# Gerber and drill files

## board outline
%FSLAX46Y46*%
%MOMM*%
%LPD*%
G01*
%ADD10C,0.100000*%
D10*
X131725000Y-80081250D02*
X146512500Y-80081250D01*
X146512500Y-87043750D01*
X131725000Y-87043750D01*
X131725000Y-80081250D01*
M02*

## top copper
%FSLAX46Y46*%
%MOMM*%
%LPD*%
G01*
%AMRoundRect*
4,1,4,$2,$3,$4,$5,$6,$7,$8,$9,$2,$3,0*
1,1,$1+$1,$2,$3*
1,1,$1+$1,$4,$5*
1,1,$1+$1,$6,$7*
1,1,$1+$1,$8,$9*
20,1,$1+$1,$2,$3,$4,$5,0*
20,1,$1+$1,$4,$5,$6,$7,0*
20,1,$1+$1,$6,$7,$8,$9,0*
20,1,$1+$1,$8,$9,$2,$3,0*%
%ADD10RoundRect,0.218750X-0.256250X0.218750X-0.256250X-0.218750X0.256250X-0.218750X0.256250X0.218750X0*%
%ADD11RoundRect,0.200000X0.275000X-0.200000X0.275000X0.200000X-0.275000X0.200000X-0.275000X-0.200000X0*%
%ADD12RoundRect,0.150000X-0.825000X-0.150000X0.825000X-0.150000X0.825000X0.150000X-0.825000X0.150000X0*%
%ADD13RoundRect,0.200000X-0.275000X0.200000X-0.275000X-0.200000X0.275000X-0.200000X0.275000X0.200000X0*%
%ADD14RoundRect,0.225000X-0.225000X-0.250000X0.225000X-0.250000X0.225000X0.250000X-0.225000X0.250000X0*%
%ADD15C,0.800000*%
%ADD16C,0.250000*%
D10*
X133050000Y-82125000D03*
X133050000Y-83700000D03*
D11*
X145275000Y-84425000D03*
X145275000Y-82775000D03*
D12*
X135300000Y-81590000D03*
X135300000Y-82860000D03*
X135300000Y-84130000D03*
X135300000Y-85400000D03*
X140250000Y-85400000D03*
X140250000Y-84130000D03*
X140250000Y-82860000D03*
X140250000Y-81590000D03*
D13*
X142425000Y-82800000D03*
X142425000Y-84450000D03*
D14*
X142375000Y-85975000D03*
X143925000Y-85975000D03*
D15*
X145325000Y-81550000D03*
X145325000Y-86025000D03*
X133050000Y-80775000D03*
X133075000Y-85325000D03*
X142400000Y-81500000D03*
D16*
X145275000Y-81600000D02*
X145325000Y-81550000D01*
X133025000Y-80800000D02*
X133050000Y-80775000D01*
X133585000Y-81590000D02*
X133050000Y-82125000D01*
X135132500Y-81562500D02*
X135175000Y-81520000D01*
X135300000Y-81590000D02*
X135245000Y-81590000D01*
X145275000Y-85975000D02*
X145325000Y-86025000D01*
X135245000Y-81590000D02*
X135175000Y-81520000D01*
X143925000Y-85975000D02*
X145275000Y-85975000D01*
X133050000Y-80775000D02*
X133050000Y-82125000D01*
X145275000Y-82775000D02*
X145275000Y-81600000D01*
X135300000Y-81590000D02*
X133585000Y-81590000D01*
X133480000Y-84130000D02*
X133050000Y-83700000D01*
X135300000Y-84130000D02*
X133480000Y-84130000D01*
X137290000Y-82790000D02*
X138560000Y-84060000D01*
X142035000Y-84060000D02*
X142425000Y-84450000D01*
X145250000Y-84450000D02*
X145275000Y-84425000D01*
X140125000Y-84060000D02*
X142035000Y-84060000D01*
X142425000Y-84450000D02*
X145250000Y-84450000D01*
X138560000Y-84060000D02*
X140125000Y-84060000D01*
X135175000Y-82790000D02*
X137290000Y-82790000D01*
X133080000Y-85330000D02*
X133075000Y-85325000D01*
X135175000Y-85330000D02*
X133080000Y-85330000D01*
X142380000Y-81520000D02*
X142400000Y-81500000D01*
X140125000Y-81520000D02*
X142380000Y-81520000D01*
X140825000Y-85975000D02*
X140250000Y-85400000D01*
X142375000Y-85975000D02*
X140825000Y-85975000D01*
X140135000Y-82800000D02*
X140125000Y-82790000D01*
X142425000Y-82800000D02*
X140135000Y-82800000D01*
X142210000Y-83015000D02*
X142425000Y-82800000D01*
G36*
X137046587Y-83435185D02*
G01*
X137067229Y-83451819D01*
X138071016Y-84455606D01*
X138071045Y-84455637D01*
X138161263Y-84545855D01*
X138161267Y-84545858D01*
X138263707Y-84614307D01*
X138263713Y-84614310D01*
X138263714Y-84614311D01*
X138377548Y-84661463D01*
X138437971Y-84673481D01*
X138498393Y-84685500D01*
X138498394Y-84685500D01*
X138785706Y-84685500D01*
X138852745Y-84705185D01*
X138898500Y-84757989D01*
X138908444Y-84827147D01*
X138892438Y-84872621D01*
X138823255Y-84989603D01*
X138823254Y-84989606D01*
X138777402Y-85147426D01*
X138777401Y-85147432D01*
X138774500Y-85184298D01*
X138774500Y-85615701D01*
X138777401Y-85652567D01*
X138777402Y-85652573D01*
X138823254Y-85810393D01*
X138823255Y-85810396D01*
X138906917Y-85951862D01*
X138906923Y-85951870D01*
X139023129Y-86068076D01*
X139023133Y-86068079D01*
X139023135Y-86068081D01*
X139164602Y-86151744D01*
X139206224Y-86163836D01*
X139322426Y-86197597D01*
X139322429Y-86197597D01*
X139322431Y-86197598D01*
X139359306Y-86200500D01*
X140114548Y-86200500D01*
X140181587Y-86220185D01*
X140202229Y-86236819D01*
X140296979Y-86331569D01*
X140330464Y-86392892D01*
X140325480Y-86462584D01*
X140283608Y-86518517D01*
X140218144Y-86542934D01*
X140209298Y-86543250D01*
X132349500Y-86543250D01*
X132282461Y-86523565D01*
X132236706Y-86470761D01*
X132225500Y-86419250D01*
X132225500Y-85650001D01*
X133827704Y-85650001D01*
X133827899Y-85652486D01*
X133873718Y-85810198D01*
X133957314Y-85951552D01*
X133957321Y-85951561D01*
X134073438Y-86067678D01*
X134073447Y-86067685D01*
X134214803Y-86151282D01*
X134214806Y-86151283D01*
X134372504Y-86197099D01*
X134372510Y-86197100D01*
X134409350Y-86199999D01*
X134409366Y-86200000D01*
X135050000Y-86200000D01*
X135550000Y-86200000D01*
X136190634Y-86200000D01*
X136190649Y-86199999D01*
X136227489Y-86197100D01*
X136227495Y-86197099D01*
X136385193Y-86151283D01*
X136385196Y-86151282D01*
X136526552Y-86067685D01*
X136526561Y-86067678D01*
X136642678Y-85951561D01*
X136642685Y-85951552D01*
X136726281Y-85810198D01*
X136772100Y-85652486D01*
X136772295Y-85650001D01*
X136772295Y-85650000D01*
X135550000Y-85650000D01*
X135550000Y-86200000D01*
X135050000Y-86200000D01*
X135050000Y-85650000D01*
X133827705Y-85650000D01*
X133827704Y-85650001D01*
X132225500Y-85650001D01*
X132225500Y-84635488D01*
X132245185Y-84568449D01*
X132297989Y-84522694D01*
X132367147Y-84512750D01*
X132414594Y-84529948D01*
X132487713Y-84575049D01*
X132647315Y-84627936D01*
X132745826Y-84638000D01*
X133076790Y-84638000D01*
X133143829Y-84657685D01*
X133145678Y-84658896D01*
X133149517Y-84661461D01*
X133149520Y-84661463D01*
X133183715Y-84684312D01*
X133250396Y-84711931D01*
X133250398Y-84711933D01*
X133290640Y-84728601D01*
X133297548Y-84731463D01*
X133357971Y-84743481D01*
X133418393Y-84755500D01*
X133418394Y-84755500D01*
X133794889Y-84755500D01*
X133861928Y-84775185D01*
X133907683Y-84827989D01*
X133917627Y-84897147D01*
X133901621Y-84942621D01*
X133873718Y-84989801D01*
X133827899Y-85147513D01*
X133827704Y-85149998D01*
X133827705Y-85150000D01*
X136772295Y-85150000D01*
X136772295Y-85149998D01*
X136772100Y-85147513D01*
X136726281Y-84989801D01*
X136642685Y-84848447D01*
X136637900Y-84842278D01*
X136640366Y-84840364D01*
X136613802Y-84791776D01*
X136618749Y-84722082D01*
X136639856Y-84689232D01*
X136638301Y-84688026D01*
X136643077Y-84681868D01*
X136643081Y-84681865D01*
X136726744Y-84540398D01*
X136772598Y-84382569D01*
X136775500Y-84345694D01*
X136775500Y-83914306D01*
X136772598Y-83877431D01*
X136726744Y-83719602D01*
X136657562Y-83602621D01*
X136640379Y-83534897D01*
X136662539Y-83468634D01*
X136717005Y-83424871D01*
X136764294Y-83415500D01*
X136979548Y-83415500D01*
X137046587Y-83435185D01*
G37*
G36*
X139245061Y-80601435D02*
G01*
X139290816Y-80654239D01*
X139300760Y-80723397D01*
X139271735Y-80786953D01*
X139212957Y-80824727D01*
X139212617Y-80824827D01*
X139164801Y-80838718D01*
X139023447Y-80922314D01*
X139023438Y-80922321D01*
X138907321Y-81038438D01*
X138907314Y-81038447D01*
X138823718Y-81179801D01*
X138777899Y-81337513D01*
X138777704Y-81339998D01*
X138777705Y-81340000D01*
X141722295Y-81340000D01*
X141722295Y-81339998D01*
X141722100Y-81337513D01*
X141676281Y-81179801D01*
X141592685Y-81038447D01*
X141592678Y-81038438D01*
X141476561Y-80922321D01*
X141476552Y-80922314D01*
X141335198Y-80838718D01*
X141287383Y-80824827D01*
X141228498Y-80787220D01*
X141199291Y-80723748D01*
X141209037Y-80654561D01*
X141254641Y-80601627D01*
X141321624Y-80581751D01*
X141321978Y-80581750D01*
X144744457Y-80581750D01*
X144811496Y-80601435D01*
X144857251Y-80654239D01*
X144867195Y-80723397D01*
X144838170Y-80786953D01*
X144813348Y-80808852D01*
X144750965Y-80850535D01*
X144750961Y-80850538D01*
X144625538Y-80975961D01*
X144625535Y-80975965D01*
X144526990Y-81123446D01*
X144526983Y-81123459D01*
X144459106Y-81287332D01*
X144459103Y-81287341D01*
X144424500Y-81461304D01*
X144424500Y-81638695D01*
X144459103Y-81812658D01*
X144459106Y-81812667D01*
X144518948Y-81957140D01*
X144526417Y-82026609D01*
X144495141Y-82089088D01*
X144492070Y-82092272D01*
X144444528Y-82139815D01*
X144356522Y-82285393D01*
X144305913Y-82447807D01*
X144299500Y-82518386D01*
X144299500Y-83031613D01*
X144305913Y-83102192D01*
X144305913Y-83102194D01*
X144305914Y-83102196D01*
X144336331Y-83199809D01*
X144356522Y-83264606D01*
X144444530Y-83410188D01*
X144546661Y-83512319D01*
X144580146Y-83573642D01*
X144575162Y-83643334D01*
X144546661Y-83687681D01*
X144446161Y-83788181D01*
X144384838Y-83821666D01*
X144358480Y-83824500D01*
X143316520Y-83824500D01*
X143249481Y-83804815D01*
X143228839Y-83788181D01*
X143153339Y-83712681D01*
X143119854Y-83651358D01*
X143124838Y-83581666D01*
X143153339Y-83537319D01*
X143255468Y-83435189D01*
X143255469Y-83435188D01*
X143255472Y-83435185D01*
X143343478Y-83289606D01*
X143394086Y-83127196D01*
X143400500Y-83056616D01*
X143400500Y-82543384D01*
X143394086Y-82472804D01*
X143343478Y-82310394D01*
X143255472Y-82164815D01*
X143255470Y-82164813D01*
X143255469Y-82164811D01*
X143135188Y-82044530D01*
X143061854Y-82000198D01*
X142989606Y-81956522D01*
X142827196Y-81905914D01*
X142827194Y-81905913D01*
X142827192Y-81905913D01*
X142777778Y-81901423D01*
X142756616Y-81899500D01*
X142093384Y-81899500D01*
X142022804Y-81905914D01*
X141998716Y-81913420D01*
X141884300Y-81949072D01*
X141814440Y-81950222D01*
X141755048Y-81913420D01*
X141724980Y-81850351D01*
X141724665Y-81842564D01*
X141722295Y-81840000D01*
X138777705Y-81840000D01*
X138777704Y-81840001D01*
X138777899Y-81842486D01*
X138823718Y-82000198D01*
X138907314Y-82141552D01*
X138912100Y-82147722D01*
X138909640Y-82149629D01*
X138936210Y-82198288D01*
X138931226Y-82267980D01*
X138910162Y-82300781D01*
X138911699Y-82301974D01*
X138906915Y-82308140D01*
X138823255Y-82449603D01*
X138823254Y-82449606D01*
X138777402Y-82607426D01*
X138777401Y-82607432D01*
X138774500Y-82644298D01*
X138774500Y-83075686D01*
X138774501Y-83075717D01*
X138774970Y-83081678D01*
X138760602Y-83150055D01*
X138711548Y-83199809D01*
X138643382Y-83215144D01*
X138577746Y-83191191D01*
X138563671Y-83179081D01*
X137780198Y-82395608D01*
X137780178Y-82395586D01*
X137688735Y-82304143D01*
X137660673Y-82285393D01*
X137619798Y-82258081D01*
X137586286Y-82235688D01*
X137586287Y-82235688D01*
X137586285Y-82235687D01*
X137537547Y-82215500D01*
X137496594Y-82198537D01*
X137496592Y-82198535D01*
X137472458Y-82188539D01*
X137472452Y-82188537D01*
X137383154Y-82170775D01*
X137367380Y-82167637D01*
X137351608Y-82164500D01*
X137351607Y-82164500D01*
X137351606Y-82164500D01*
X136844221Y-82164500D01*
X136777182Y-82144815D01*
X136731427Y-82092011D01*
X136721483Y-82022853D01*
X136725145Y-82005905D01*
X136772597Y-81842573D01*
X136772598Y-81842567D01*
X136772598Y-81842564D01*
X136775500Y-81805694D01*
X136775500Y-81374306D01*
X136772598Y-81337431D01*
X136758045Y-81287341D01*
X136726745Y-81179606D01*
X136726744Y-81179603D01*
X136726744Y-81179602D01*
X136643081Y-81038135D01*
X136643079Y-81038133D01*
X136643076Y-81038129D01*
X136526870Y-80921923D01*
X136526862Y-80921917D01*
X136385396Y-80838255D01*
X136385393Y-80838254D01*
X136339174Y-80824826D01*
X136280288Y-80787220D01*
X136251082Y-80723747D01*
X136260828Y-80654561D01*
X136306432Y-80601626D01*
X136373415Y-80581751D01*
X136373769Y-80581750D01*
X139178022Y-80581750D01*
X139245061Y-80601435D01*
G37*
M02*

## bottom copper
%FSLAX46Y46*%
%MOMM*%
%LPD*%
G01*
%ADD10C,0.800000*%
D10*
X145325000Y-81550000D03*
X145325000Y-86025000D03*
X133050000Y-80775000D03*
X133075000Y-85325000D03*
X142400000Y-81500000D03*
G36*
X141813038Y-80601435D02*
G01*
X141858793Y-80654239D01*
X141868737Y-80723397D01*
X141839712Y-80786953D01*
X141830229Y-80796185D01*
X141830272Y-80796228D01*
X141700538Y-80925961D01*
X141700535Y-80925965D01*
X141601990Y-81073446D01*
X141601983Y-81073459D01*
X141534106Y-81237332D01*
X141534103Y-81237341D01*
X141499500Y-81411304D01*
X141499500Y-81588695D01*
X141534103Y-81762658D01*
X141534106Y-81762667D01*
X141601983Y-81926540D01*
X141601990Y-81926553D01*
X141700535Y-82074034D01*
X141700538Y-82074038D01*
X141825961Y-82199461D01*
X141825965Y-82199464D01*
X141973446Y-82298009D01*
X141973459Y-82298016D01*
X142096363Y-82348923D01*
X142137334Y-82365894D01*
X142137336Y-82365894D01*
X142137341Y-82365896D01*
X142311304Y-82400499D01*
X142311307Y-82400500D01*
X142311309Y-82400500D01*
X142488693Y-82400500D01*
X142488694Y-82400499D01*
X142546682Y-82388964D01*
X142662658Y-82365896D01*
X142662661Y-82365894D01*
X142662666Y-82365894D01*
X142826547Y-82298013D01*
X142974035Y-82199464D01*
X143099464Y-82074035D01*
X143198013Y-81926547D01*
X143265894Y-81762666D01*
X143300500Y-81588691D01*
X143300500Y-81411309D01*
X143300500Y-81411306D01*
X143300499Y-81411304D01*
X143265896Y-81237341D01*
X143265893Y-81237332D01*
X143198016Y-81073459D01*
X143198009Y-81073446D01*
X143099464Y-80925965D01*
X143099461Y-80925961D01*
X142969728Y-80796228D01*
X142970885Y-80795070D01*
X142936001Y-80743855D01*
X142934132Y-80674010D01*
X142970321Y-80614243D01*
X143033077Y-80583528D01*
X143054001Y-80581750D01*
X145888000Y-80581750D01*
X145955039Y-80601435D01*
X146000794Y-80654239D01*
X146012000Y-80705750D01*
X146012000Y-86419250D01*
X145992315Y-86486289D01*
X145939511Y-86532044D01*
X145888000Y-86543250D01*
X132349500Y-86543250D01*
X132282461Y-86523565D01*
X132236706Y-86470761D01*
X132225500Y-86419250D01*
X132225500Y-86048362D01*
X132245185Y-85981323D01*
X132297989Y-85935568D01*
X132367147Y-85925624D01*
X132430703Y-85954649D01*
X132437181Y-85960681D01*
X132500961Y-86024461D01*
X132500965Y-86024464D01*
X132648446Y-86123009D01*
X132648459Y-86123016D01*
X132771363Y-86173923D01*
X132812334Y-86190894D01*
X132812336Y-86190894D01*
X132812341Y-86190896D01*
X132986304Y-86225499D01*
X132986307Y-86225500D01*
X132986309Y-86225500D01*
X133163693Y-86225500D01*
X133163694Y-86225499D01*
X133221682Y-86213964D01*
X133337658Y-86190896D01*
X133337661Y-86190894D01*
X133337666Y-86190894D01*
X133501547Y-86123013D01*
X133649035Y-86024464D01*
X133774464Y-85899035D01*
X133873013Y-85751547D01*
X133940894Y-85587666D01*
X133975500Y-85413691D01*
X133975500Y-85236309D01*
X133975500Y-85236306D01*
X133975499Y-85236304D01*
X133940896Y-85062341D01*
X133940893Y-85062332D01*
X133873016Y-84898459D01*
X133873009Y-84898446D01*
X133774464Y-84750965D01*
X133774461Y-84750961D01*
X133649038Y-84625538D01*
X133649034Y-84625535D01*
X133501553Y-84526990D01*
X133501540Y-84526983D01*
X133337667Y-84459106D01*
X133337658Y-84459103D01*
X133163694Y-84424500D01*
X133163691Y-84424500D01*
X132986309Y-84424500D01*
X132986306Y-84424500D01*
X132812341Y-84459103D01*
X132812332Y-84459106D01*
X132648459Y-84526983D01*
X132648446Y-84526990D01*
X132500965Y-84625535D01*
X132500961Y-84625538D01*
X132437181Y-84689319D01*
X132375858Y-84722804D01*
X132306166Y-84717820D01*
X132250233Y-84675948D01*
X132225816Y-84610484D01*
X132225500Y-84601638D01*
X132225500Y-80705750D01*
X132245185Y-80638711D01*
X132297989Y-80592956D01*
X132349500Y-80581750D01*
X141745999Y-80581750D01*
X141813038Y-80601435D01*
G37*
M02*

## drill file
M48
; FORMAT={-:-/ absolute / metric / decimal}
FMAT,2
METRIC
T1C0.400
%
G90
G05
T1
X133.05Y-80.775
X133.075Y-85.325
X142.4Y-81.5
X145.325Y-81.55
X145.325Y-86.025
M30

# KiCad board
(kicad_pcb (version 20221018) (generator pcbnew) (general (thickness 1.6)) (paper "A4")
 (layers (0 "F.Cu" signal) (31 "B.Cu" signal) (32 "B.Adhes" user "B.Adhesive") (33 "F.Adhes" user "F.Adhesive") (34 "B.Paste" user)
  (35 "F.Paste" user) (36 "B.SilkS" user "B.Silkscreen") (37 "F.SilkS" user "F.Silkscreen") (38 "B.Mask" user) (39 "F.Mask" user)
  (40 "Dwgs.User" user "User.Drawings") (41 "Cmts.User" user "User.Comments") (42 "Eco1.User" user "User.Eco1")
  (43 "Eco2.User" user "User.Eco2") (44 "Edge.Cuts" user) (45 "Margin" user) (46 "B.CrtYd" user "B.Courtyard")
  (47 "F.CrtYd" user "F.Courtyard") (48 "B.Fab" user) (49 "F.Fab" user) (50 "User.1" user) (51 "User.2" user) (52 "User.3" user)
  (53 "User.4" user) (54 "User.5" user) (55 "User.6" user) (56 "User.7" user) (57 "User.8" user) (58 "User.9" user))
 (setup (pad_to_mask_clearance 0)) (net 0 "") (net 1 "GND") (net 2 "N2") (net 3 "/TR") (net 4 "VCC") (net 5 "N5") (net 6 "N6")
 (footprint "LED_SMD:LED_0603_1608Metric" (layer "F.Cu") (at 133.05 82.9125 -90)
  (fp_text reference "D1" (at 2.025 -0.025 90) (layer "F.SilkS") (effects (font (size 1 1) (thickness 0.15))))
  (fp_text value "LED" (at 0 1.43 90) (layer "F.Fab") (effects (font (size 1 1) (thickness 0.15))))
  (pad "1" smd roundrect (at -0.7875 0 270) (size 0.875 0.95) (layers "F.Cu" "F.Paste" "F.Mask") (roundrect_rratio 0.25) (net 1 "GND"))
  (pad "2" smd roundrect (at 0.7875 0 270) (size 0.875 0.95) (layers "F.Cu" "F.Paste" "F.Mask") (roundrect_rratio 0.25) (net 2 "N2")))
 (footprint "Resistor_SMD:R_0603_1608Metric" (layer "F.Cu") (at 145.275 83.6 90)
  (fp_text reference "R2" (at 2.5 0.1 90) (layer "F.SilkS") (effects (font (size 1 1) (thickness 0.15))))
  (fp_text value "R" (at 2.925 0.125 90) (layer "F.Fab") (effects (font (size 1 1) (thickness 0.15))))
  (pad "1" smd roundrect (at -0.825 0 90) (size 0.8 0.95) (layers "F.Cu" "F.Paste" "F.Mask") (roundrect_rratio 0.25) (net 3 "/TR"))
  (pad "2" smd roundrect (at 0.825 0 90) (size 0.8 0.95) (layers "F.Cu" "F.Paste" "F.Mask") (roundrect_rratio 0.25) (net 1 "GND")))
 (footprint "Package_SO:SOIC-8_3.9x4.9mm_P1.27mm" (layer "F.Cu") (at 137.775 83.495)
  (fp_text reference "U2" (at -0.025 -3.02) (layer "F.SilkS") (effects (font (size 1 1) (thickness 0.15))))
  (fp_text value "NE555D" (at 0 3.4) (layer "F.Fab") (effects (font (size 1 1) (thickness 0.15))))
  (pad "1" smd roundrect (at -2.475 -1.905) (size 1.95 0.6) (layers "F.Cu" "F.Paste" "F.Mask") (roundrect_rratio 0.25) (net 1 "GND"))
  (pad "2" smd roundrect (at -2.475 -0.635) (size 1.95 0.6) (layers "F.Cu" "F.Paste" "F.Mask") (roundrect_rratio 0.25) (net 3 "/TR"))
  (pad "3" smd roundrect (at -2.475 0.635) (size 1.95 0.6) (layers "F.Cu" "F.Paste" "F.Mask") (roundrect_rratio 0.25) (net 2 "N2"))
  (pad "4" smd roundrect (at -2.475 1.905) (size 1.95 0.6) (layers "F.Cu" "F.Paste" "F.Mask") (roundrect_rratio 0.25) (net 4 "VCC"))
  (pad "5" smd roundrect (at 2.475 1.905) (size 1.95 0.6) (layers "F.Cu" "F.Paste" "F.Mask") (roundrect_rratio 0.25) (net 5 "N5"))
  (pad "6" smd roundrect (at 2.475 0.635) (size 1.95 0.6) (layers "F.Cu" "F.Paste" "F.Mask") (roundrect_rratio 0.25) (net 3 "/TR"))
  (pad "7" smd roundrect (at 2.475 -0.635) (size 1.95 0.6) (layers "F.Cu" "F.Paste" "F.Mask") (roundrect_rratio 0.25) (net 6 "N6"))
  (pad "8" smd roundrect (at 2.475 -1.905) (size 1.95 0.6) (layers "F.Cu" "F.Paste" "F.Mask") (roundrect_rratio 0.25) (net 4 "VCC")))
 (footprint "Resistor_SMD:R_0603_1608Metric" (layer "F.Cu") (at 142.425 83.625 -90)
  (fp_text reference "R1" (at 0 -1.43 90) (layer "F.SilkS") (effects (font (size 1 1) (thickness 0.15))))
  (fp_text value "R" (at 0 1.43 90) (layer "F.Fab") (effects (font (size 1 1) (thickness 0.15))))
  (pad "1" smd roundrect (at -0.825 0 270) (size 0.8 0.95) (layers "F.Cu" "F.Paste" "F.Mask") (roundrect_rratio 0.25) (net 6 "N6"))
  (pad "2" smd roundrect (at 0.825 0 270) (size 0.8 0.95) (layers "F.Cu" "F.Paste" "F.Mask") (roundrect_rratio 0.25) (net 3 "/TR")))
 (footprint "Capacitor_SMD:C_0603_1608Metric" (layer "F.Cu") (at 143.15 85.975)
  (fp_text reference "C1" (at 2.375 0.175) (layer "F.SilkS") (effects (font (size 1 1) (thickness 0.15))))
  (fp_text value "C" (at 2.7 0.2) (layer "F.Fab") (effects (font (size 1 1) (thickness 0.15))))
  (pad "1" smd roundrect (at -0.775 0) (size 0.9 0.95) (layers "F.Cu" "F.Paste" "F.Mask") (roundrect_rratio 0.25) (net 5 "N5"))
  (pad "2" smd roundrect (at 0.775 0) (size 0.9 0.95) (layers "F.Cu" "F.Paste" "F.Mask") (roundrect_rratio 0.25) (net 1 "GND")))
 (gr_rect (start 131.725 80.08125) (end 146.5125 87.04375) (stroke (width 0.1) (type default)) (fill none) (layer "Edge.Cuts"))
 (segment (start 145.275 81.6) (end 145.325 81.55) (width 0.25) (layer "F.Cu") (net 1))
 (segment (start 133.025 80.8) (end 133.05 80.775) (width 0.25) (layer "F.Cu") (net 1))
 (segment (start 133.585 81.59) (end 133.05 82.125) (width 0.25) (layer "F.Cu") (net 1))
 (segment (start 135.1325 81.5625) (end 135.175 81.52) (width 0.25) (layer "F.Cu") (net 1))
 (segment (start 135.3 81.59) (end 135.245 81.59) (width 0.25) (layer "F.Cu") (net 1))
 (segment (start 145.275 85.975) (end 145.325 86.025) (width 0.25) (layer "F.Cu") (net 1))
 (segment (start 135.245 81.59) (end 135.175 81.52) (width 0.25) (layer "F.Cu") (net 1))
 (segment (start 143.925 85.975) (end 145.275 85.975) (width 0.25) (layer "F.Cu") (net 1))
 (segment (start 133.05 80.775) (end 133.05 82.125) (width 0.25) (layer "F.Cu") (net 1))
 (segment (start 145.275 82.775) (end 145.275 81.6) (width 0.25) (layer "F.Cu") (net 1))
 (segment (start 135.3 81.59) (end 133.585 81.59) (width 0.25) (layer "F.Cu") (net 1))
 (via (at 145.325 81.55) (size 0.8) (drill 0.4) (layers "F.Cu" "B.Cu") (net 1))
 (via (at 145.325 86.025) (size 0.8) (drill 0.4) (layers "F.Cu" "B.Cu") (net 1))
 (via (at 133.05 80.775) (size 0.8) (drill 0.4) (layers "F.Cu" "B.Cu") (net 1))
 (segment (start 133.48 84.13) (end 133.05 83.7) (width 0.25) (layer "F.Cu") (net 2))
 (segment (start 135.3 84.13) (end 133.48 84.13) (width 0.25) (layer "F.Cu") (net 2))
 (segment (start 137.29 82.79) (end 138.56 84.06) (width 0.25) (layer "F.Cu") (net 3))
 (segment (start 142.035 84.06) (end 142.425 84.45) (width 0.25) (layer "F.Cu") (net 3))
 (segment (start 145.25 84.45) (end 145.275 84.425) (width 0.25) (layer "F.Cu") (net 3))
 (segment (start 140.125 84.06) (end 142.035 84.06) (width 0.25) (layer "F.Cu") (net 3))
 (segment (start 142.425 84.45) (end 145.25 84.45) (width 0.25) (layer "F.Cu") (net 3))
 (segment (start 138.56 84.06) (end 140.125 84.06) (width 0.25) (layer "F.Cu") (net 3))
 (segment (start 135.175 82.79) (end 137.29 82.79) (width 0.25) (layer "F.Cu") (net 3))
 (segment (start 133.08 85.33) (end 133.075 85.325) (width 0.25) (layer "F.Cu") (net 4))
 (segment (start 135.175 85.33) (end 133.08 85.33) (width 0.25) (layer "F.Cu") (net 4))
 (segment (start 142.38 81.52) (end 142.4 81.5) (width 0.25) (layer "F.Cu") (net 4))
 (segment (start 140.125 81.52) (end 142.38 81.52) (width 0.25) (layer "F.Cu") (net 4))
 (via (at 133.075 85.325) (size 0.8) (drill 0.4) (layers "F.Cu" "B.Cu") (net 4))
 (via (at 142.4 81.5) (size 0.8) (drill 0.4) (layers "F.Cu" "B.Cu") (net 4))
 (segment (start 140.825 85.975) (end 140.25 85.4) (width 0.25) (layer "F.Cu") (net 5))
 (segment (start 142.375 85.975) (end 140.825 85.975) (width 0.25) (layer "F.Cu") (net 5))
 (segment (start 140.135 82.8) (end 140.125 82.79) (width 0.25) (layer "F.Cu") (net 6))
 (segment (start 142.425 82.8) (end 140.135 82.8) (width 0.25) (layer "F.Cu") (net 6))
 (segment (start 142.21 83.015) (end 142.425 82.8) (width 0.25) (layer "F.Cu") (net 6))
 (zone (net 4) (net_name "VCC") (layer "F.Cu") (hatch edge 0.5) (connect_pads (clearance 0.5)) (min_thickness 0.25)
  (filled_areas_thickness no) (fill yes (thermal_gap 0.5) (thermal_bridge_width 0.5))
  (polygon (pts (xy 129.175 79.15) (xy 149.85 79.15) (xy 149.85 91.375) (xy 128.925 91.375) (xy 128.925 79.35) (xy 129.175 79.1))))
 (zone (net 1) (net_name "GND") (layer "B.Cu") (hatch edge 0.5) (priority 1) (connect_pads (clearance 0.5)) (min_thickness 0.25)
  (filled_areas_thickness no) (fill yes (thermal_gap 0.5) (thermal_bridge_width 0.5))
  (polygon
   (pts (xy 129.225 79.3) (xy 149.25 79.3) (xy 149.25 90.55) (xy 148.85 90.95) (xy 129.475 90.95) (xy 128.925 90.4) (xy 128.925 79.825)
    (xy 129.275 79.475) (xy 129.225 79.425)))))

